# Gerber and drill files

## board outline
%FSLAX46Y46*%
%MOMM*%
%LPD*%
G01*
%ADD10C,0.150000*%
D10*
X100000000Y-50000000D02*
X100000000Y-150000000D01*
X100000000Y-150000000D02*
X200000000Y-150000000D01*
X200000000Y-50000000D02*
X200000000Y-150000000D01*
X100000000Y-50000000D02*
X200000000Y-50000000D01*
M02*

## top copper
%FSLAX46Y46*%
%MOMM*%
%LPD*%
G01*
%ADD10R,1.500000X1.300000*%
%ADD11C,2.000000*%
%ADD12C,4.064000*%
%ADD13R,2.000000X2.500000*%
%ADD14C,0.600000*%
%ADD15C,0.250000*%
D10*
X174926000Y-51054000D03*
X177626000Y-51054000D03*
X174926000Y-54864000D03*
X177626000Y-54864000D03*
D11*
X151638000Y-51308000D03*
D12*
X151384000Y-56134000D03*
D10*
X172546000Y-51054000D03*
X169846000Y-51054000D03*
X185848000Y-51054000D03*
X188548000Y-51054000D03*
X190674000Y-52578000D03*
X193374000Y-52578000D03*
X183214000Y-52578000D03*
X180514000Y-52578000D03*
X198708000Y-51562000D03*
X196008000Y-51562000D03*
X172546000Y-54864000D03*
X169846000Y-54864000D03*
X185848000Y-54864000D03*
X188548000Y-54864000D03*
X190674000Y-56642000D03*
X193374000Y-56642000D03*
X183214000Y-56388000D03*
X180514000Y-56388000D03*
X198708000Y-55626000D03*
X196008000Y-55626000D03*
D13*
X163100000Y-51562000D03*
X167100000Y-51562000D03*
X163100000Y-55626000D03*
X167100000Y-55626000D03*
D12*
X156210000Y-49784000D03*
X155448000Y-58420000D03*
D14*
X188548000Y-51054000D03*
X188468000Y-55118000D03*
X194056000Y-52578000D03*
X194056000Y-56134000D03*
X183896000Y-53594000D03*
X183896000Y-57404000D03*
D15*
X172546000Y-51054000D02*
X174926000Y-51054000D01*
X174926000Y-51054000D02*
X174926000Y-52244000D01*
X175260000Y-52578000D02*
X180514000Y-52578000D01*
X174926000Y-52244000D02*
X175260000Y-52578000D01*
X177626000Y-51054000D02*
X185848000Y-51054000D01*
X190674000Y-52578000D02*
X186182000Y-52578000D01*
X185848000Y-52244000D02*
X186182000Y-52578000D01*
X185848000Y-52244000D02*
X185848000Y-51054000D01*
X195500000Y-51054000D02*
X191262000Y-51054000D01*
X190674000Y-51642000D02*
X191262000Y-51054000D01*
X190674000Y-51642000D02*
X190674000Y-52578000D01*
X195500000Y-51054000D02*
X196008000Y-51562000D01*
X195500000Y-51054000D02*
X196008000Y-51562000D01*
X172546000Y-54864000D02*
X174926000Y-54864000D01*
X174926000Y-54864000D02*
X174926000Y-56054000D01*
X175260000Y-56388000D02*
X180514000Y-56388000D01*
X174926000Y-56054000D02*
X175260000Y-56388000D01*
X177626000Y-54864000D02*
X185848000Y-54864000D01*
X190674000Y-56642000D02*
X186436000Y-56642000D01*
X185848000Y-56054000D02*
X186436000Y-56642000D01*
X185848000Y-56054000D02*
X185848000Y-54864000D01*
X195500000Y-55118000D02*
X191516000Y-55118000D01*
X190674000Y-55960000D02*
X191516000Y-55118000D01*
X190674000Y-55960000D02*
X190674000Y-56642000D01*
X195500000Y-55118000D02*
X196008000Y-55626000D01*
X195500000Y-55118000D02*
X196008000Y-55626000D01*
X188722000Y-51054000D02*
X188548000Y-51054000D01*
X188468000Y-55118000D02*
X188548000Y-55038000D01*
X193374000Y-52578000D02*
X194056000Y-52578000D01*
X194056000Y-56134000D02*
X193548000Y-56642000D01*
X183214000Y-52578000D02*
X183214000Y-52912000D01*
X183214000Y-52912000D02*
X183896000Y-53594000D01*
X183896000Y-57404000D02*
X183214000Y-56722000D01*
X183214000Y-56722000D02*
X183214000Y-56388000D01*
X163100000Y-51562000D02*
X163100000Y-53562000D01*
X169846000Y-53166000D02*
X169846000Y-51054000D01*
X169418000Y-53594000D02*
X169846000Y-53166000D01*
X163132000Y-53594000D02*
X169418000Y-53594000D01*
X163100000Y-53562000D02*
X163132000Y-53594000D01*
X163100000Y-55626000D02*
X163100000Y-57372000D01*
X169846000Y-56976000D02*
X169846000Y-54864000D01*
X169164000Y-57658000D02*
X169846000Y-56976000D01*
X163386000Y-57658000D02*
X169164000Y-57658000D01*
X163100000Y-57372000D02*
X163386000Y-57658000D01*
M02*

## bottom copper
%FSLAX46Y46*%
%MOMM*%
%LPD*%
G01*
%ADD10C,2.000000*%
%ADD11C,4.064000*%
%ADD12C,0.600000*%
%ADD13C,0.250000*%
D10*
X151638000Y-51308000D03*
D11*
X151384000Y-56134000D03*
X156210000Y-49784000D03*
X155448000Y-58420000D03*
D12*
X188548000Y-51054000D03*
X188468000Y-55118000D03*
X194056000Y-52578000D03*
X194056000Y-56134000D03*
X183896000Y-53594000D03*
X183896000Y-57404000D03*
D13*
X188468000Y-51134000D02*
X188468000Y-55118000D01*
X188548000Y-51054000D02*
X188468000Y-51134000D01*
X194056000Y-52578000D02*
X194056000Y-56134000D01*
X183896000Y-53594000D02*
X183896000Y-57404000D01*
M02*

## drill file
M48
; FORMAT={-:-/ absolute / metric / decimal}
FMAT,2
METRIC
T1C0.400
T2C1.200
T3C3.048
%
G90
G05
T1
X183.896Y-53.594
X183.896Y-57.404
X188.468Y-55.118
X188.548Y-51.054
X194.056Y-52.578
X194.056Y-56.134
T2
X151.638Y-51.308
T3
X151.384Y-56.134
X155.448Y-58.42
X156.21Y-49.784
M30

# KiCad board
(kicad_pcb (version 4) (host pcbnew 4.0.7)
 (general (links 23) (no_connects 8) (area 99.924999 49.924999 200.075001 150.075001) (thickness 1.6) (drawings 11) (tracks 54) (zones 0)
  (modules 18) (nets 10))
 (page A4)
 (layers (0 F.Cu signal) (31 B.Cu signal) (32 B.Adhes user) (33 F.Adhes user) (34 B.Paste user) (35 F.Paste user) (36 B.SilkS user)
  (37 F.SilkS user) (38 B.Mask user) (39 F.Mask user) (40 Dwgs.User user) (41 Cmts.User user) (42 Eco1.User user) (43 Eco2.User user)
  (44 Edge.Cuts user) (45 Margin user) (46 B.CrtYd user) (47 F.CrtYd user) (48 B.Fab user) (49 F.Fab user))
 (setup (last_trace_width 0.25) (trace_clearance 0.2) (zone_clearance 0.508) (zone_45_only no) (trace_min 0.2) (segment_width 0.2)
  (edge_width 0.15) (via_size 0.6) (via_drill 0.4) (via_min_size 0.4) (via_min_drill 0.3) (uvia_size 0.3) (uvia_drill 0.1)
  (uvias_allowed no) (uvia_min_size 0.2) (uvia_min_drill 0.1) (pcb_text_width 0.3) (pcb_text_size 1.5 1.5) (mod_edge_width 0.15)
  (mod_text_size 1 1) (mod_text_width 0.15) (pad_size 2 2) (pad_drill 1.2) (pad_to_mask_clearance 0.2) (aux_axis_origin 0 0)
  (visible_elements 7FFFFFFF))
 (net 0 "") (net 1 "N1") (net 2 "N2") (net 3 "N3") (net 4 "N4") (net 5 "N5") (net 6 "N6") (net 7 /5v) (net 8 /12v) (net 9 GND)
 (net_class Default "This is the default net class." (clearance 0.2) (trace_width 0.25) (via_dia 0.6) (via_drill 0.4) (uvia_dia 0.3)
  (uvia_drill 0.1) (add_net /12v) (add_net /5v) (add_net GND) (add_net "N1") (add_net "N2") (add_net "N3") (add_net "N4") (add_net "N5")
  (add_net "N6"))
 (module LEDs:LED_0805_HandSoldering (layer F.Cu) (at 176.276 51.054)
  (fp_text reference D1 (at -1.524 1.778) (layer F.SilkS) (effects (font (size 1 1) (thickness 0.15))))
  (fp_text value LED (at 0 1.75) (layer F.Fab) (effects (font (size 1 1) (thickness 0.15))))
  (pad 1 smd rect (at -1.35 0) (size 1.5 1.3) (layers F.Cu F.Paste F.Mask) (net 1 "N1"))
  (pad 2 smd rect (at 1.35 0) (size 1.5 1.3) (layers F.Cu F.Paste F.Mask) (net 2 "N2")))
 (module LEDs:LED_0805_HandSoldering (layer F.Cu) (at 176.276 54.864)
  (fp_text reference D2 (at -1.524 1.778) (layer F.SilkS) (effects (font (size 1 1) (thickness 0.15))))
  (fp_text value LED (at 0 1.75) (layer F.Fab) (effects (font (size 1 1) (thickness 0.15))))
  (pad 1 smd rect (at -1.35 0) (size 1.5 1.3) (layers F.Cu F.Paste F.Mask) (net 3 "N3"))
  (pad 2 smd rect (at 1.35 0) (size 1.5 1.3) (layers F.Cu F.Paste F.Mask) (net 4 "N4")))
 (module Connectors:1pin (layer F.Cu) (at 151.638 51.308)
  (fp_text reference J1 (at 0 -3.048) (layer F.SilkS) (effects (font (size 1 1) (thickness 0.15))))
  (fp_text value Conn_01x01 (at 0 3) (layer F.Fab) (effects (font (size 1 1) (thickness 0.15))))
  (pad 1 thru_hole circle (at 0 0) (size 2 2) (drill 1.2) (layers *.Cu *.Mask) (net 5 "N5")))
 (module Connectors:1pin (layer F.Cu) (at 151.384 56.134)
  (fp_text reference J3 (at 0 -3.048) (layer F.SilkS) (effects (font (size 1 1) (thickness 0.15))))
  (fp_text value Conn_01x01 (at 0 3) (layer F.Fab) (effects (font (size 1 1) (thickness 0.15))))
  (pad 1 thru_hole circle (at 0 0) (size 4.064 4.064) (drill 3.048) (layers *.Cu *.Mask) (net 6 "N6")))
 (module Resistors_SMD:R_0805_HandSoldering (layer F.Cu) (at 171.196 51.054 180)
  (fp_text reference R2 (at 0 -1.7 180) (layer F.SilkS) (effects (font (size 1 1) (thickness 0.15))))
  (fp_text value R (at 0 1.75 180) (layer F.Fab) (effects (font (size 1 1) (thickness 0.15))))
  (pad 1 smd rect (at -1.35 0 180) (size 1.5 1.3) (layers F.Cu F.Paste F.Mask) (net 1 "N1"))
  (pad 2 smd rect (at 1.35 0 180) (size 1.5 1.3) (layers F.Cu F.Paste F.Mask) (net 5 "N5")))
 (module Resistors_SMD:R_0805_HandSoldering (layer F.Cu) (at 187.198 51.054)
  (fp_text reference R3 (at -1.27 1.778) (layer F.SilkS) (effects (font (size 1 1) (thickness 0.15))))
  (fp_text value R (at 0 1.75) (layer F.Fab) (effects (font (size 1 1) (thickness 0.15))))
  (pad 1 smd rect (at -1.35 0) (size 1.5 1.3) (layers F.Cu F.Paste F.Mask) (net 2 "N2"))
  (pad 2 smd rect (at 1.35 0) (size 1.5 1.3) (layers F.Cu F.Paste F.Mask) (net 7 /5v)))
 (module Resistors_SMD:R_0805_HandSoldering (layer F.Cu) (at 192.024 52.578)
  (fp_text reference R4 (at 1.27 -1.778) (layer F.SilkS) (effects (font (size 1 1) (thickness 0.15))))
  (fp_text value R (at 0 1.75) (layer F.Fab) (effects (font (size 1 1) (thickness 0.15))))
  (pad 1 smd rect (at -1.35 0) (size 1.5 1.3) (layers F.Cu F.Paste F.Mask) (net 2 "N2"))
  (pad 2 smd rect (at 1.35 0) (size 1.5 1.3) (layers F.Cu F.Paste F.Mask) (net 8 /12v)))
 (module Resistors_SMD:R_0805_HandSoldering (layer F.Cu) (at 181.864 52.578 180)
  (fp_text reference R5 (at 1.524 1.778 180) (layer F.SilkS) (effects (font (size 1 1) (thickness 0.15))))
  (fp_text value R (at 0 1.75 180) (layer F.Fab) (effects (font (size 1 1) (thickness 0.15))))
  (pad 1 smd rect (at -1.35 0 180) (size 1.5 1.3) (layers F.Cu F.Paste F.Mask) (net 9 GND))
  (pad 2 smd rect (at 1.35 0 180) (size 1.5 1.3) (layers F.Cu F.Paste F.Mask) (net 1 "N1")))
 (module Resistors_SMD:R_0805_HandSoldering (layer F.Cu) (at 197.358 51.562 180)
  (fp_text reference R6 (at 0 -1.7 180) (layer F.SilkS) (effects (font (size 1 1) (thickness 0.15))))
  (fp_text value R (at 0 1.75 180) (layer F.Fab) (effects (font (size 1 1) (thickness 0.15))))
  (pad 1 smd rect (at -1.35 0 180) (size 1.5 1.3) (layers F.Cu F.Paste F.Mask) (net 9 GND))
  (pad 2 smd rect (at 1.35 0 180) (size 1.5 1.3) (layers F.Cu F.Paste F.Mask) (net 2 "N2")))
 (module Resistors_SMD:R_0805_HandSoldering (layer F.Cu) (at 171.196 54.864 180)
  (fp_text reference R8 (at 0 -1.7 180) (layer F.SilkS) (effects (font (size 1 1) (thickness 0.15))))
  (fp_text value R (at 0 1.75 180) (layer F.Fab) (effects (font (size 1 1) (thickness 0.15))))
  (pad 1 smd rect (at -1.35 0 180) (size 1.5 1.3) (layers F.Cu F.Paste F.Mask) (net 3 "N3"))
  (pad 2 smd rect (at 1.35 0 180) (size 1.5 1.3) (layers F.Cu F.Paste F.Mask) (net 6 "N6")))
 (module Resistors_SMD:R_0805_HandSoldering (layer F.Cu) (at 187.198 54.864)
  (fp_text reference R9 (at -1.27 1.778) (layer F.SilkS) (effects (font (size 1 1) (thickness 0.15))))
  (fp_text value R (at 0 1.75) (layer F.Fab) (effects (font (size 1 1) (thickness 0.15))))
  (pad 1 smd rect (at -1.35 0) (size 1.5 1.3) (layers F.Cu F.Paste F.Mask) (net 4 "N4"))
  (pad 2 smd rect (at 1.35 0) (size 1.5 1.3) (layers F.Cu F.Paste F.Mask) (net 7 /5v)))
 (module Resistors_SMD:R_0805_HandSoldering (layer F.Cu) (at 192.024 56.642)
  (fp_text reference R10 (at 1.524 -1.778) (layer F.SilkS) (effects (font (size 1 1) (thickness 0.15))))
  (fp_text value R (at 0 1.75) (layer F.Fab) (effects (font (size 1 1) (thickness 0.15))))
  (pad 1 smd rect (at -1.35 0) (size 1.5 1.3) (layers F.Cu F.Paste F.Mask) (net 4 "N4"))
  (pad 2 smd rect (at 1.35 0) (size 1.5 1.3) (layers F.Cu F.Paste F.Mask) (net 8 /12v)))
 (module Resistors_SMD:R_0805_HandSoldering (layer F.Cu) (at 181.864 56.388 180)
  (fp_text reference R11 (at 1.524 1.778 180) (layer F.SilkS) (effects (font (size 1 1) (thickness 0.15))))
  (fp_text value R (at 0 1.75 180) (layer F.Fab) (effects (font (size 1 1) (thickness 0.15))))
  (pad 1 smd rect (at -1.35 0 180) (size 1.5 1.3) (layers F.Cu F.Paste F.Mask) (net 9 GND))
  (pad 2 smd rect (at 1.35 0 180) (size 1.5 1.3) (layers F.Cu F.Paste F.Mask) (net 3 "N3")))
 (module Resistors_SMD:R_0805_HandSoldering (layer F.Cu) (at 197.358 55.626 180)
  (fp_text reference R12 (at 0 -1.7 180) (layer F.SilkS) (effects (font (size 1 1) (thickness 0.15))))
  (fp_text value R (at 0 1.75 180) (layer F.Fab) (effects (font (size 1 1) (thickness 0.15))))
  (pad 1 smd rect (at -1.35 0 180) (size 1.5 1.3) (layers F.Cu F.Paste F.Mask) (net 9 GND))
  (pad 2 smd rect (at 1.35 0 180) (size 1.5 1.3) (layers F.Cu F.Paste F.Mask) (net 4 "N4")))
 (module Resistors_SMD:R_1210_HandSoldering (layer F.Cu) (at 165.1 51.562)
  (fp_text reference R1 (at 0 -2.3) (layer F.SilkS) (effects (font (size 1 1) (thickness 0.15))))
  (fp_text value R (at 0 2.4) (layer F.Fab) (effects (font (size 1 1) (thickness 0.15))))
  (pad 1 smd rect (at -2 0) (size 2 2.5) (layers F.Cu F.Paste F.Mask) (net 5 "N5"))
  (pad 2 smd rect (at 2 0) (size 2 2.5) (layers F.Cu F.Paste F.Mask) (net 9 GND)))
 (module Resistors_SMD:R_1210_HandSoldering (layer F.Cu) (at 165.1 55.626)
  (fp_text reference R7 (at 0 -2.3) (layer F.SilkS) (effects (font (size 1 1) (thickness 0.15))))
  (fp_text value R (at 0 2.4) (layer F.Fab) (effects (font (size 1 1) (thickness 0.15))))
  (pad 1 smd rect (at -2 0) (size 2 2.5) (layers F.Cu F.Paste F.Mask) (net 6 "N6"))
  (pad 2 smd rect (at 2 0) (size 2 2.5) (layers F.Cu F.Paste F.Mask) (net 9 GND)))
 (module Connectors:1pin (layer F.Cu) (at 156.21 49.784)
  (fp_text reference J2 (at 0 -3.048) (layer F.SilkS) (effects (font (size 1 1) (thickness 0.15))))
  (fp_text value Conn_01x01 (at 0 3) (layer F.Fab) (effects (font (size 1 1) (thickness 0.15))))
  (pad 1 thru_hole circle (at 0 0) (size 4.064 4.064) (drill 3.048) (layers *.Cu *.Mask) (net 5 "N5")))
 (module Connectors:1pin (layer F.Cu) (at 155.448 58.42)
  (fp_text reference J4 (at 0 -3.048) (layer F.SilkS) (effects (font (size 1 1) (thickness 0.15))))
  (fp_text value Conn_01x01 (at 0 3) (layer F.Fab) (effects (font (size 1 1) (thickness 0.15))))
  (pad 1 thru_hole circle (at 0 0) (size 4.064 4.064) (drill 3.048) (layers *.Cu *.Mask) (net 6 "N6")))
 (gr_line (start 100 50) (end 100 150) (angle 90) (layer Edge.Cuts) (width 0.15))
 (gr_line (start 100 150) (end 200 150) (angle 90) (layer Edge.Cuts) (width 0.15))
 (gr_line (start 200 50) (end 200 150) (angle 90) (layer Edge.Cuts) (width 0.15))
 (gr_line (start 100 50) (end 200 50) (angle 90) (layer Edge.Cuts) (width 0.15))
 (segment (start 172.546 51.054) (end 174.926 51.054) (width 0.25) (layer F.Cu) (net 1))
 (segment (start 174.926 51.054) (end 174.926 52.244) (width 0.25) (layer F.Cu) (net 1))
 (segment (start 175.26 52.578) (end 180.514 52.578) (width 0.25) (layer F.Cu) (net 1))
 (segment (start 174.926 52.244) (end 175.26 52.578) (width 0.25) (layer F.Cu) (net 1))
 (segment (start 177.626 51.054) (end 185.848 51.054) (width 0.25) (layer F.Cu) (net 2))
 (segment (start 190.674 52.578) (end 186.182 52.578) (width 0.25) (layer F.Cu) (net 2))
 (segment (start 185.848 52.244) (end 186.182 52.578) (width 0.25) (layer F.Cu) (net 2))
 (segment (start 185.848 52.244) (end 185.848 51.054) (width 0.25) (layer F.Cu) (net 2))
 (segment (start 195.5 51.054) (end 191.262 51.054) (width 0.25) (layer F.Cu) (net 2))
 (segment (start 190.674 51.642) (end 191.262 51.054) (width 0.25) (layer F.Cu) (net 2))
 (segment (start 190.674 51.642) (end 190.674 52.578) (width 0.25) (layer F.Cu) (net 2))
 (segment (start 195.5 51.054) (end 196.008 51.562) (width 0.25) (layer F.Cu) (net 2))
 (segment (start 195.5 51.054) (end 196.008 51.562) (width 0.25) (layer F.Cu) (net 2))
 (segment (start 172.546 54.864) (end 174.926 54.864) (width 0.25) (layer F.Cu) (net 3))
 (segment (start 174.926 54.864) (end 174.926 56.054) (width 0.25) (layer F.Cu) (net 3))
 (segment (start 175.26 56.388) (end 180.514 56.388) (width 0.25) (layer F.Cu) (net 3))
 (segment (start 174.926 56.054) (end 175.26 56.388) (width 0.25) (layer F.Cu) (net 3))
 (segment (start 177.626 54.864) (end 185.848 54.864) (width 0.25) (layer F.Cu) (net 4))
 (segment (start 190.674 56.642) (end 186.436 56.642) (width 0.25) (layer F.Cu) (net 4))
 (segment (start 185.848 56.054) (end 186.436 56.642) (width 0.25) (layer F.Cu) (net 4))
 (segment (start 185.848 56.054) (end 185.848 54.864) (width 0.25) (layer F.Cu) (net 4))
 (segment (start 195.5 55.118) (end 191.516 55.118) (width 0.25) (layer F.Cu) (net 4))
 (segment (start 190.674 55.96) (end 191.516 55.118) (width 0.25) (layer F.Cu) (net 4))
 (segment (start 190.674 55.96) (end 190.674 56.642) (width 0.25) (layer F.Cu) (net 4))
 (segment (start 195.5 55.118) (end 196.008 55.626) (width 0.25) (layer F.Cu) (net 4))
 (segment (start 195.5 55.118) (end 196.008 55.626) (width 0.25) (layer F.Cu) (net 4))
 (via (at 188.548 51.054) (size 0.6) (drill 0.4) (layers F.Cu B.Cu) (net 7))
 (segment (start 188.722 51.054) (end 188.548 51.054) (width 0.25) (layer F.Cu) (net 7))
 (segment (start 188.468 55.118) (end 188.548 55.038) (width 0.25) (layer F.Cu) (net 7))
 (via (at 188.468 55.118) (size 0.6) (drill 0.4) (layers F.Cu B.Cu) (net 7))
 (segment (start 188.468 51.134) (end 188.468 55.118) (width 0.25) (layer B.Cu) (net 7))
 (segment (start 188.548 51.054) (end 188.468 51.134) (width 0.25) (layer B.Cu) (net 7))
 (segment (start 193.374 52.578) (end 194.056 52.578) (width 0.25) (layer F.Cu) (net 8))
 (via (at 194.056 52.578) (size 0.6) (drill 0.4) (layers F.Cu B.Cu) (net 8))
 (segment (start 194.056 52.578) (end 194.056 56.134) (width 0.25) (layer B.Cu) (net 8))
 (via (at 194.056 56.134) (size 0.6) (drill 0.4) (layers F.Cu B.Cu) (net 8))
 (segment (start 194.056 56.134) (end 193.548 56.642) (width 0.25) (layer F.Cu) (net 8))
 (segment (start 183.214 52.578) (end 183.214 52.912) (width 0.25) (layer F.Cu) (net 9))
 (segment (start 183.214 52.912) (end 183.896 53.594) (width 0.25) (layer F.Cu) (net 9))
 (via (at 183.896 53.594) (size 0.6) (drill 0.4) (layers F.Cu B.Cu) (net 9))
 (segment (start 183.896 53.594) (end 183.896 57.404) (width 0.25) (layer B.Cu) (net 9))
 (via (at 183.896 57.404) (size 0.6) (drill 0.4) (layers F.Cu B.Cu) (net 9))
 (segment (start 183.896 57.404) (end 183.214 56.722) (width 0.25) (layer F.Cu) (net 9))
 (segment (start 183.214 56.722) (end 183.214 56.388) (width 0.25) (layer F.Cu) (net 9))
 (segment (start 163.1 51.562) (end 163.1 53.562) (width 0.25) (layer F.Cu) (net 5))
 (segment (start 169.846 53.166) (end 169.846 51.054) (width 0.25) (layer F.Cu) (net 5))
 (segment (start 169.418 53.594) (end 169.846 53.166) (width 0.25) (layer F.Cu) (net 5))
 (segment (start 163.132 53.594) (end 169.418 53.594) (width 0.25) (layer F.Cu) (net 5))
 (segment (start 163.1 53.562) (end 163.132 53.594) (width 0.25) (layer F.Cu) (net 5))
 (segment (start 163.1 55.626) (end 163.1 57.372) (width 0.25) (layer F.Cu) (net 6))
 (segment (start 169.846 56.976) (end 169.846 54.864) (width 0.25) (layer F.Cu) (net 6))
 (segment (start 169.164 57.658) (end 169.846 56.976) (width 0.25) (layer F.Cu) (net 6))
 (segment (start 163.386 57.658) (end 169.164 57.658) (width 0.25) (layer F.Cu) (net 6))
 (segment (start 163.1 57.372) (end 163.386 57.658) (width 0.25) (layer F.Cu) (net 6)))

